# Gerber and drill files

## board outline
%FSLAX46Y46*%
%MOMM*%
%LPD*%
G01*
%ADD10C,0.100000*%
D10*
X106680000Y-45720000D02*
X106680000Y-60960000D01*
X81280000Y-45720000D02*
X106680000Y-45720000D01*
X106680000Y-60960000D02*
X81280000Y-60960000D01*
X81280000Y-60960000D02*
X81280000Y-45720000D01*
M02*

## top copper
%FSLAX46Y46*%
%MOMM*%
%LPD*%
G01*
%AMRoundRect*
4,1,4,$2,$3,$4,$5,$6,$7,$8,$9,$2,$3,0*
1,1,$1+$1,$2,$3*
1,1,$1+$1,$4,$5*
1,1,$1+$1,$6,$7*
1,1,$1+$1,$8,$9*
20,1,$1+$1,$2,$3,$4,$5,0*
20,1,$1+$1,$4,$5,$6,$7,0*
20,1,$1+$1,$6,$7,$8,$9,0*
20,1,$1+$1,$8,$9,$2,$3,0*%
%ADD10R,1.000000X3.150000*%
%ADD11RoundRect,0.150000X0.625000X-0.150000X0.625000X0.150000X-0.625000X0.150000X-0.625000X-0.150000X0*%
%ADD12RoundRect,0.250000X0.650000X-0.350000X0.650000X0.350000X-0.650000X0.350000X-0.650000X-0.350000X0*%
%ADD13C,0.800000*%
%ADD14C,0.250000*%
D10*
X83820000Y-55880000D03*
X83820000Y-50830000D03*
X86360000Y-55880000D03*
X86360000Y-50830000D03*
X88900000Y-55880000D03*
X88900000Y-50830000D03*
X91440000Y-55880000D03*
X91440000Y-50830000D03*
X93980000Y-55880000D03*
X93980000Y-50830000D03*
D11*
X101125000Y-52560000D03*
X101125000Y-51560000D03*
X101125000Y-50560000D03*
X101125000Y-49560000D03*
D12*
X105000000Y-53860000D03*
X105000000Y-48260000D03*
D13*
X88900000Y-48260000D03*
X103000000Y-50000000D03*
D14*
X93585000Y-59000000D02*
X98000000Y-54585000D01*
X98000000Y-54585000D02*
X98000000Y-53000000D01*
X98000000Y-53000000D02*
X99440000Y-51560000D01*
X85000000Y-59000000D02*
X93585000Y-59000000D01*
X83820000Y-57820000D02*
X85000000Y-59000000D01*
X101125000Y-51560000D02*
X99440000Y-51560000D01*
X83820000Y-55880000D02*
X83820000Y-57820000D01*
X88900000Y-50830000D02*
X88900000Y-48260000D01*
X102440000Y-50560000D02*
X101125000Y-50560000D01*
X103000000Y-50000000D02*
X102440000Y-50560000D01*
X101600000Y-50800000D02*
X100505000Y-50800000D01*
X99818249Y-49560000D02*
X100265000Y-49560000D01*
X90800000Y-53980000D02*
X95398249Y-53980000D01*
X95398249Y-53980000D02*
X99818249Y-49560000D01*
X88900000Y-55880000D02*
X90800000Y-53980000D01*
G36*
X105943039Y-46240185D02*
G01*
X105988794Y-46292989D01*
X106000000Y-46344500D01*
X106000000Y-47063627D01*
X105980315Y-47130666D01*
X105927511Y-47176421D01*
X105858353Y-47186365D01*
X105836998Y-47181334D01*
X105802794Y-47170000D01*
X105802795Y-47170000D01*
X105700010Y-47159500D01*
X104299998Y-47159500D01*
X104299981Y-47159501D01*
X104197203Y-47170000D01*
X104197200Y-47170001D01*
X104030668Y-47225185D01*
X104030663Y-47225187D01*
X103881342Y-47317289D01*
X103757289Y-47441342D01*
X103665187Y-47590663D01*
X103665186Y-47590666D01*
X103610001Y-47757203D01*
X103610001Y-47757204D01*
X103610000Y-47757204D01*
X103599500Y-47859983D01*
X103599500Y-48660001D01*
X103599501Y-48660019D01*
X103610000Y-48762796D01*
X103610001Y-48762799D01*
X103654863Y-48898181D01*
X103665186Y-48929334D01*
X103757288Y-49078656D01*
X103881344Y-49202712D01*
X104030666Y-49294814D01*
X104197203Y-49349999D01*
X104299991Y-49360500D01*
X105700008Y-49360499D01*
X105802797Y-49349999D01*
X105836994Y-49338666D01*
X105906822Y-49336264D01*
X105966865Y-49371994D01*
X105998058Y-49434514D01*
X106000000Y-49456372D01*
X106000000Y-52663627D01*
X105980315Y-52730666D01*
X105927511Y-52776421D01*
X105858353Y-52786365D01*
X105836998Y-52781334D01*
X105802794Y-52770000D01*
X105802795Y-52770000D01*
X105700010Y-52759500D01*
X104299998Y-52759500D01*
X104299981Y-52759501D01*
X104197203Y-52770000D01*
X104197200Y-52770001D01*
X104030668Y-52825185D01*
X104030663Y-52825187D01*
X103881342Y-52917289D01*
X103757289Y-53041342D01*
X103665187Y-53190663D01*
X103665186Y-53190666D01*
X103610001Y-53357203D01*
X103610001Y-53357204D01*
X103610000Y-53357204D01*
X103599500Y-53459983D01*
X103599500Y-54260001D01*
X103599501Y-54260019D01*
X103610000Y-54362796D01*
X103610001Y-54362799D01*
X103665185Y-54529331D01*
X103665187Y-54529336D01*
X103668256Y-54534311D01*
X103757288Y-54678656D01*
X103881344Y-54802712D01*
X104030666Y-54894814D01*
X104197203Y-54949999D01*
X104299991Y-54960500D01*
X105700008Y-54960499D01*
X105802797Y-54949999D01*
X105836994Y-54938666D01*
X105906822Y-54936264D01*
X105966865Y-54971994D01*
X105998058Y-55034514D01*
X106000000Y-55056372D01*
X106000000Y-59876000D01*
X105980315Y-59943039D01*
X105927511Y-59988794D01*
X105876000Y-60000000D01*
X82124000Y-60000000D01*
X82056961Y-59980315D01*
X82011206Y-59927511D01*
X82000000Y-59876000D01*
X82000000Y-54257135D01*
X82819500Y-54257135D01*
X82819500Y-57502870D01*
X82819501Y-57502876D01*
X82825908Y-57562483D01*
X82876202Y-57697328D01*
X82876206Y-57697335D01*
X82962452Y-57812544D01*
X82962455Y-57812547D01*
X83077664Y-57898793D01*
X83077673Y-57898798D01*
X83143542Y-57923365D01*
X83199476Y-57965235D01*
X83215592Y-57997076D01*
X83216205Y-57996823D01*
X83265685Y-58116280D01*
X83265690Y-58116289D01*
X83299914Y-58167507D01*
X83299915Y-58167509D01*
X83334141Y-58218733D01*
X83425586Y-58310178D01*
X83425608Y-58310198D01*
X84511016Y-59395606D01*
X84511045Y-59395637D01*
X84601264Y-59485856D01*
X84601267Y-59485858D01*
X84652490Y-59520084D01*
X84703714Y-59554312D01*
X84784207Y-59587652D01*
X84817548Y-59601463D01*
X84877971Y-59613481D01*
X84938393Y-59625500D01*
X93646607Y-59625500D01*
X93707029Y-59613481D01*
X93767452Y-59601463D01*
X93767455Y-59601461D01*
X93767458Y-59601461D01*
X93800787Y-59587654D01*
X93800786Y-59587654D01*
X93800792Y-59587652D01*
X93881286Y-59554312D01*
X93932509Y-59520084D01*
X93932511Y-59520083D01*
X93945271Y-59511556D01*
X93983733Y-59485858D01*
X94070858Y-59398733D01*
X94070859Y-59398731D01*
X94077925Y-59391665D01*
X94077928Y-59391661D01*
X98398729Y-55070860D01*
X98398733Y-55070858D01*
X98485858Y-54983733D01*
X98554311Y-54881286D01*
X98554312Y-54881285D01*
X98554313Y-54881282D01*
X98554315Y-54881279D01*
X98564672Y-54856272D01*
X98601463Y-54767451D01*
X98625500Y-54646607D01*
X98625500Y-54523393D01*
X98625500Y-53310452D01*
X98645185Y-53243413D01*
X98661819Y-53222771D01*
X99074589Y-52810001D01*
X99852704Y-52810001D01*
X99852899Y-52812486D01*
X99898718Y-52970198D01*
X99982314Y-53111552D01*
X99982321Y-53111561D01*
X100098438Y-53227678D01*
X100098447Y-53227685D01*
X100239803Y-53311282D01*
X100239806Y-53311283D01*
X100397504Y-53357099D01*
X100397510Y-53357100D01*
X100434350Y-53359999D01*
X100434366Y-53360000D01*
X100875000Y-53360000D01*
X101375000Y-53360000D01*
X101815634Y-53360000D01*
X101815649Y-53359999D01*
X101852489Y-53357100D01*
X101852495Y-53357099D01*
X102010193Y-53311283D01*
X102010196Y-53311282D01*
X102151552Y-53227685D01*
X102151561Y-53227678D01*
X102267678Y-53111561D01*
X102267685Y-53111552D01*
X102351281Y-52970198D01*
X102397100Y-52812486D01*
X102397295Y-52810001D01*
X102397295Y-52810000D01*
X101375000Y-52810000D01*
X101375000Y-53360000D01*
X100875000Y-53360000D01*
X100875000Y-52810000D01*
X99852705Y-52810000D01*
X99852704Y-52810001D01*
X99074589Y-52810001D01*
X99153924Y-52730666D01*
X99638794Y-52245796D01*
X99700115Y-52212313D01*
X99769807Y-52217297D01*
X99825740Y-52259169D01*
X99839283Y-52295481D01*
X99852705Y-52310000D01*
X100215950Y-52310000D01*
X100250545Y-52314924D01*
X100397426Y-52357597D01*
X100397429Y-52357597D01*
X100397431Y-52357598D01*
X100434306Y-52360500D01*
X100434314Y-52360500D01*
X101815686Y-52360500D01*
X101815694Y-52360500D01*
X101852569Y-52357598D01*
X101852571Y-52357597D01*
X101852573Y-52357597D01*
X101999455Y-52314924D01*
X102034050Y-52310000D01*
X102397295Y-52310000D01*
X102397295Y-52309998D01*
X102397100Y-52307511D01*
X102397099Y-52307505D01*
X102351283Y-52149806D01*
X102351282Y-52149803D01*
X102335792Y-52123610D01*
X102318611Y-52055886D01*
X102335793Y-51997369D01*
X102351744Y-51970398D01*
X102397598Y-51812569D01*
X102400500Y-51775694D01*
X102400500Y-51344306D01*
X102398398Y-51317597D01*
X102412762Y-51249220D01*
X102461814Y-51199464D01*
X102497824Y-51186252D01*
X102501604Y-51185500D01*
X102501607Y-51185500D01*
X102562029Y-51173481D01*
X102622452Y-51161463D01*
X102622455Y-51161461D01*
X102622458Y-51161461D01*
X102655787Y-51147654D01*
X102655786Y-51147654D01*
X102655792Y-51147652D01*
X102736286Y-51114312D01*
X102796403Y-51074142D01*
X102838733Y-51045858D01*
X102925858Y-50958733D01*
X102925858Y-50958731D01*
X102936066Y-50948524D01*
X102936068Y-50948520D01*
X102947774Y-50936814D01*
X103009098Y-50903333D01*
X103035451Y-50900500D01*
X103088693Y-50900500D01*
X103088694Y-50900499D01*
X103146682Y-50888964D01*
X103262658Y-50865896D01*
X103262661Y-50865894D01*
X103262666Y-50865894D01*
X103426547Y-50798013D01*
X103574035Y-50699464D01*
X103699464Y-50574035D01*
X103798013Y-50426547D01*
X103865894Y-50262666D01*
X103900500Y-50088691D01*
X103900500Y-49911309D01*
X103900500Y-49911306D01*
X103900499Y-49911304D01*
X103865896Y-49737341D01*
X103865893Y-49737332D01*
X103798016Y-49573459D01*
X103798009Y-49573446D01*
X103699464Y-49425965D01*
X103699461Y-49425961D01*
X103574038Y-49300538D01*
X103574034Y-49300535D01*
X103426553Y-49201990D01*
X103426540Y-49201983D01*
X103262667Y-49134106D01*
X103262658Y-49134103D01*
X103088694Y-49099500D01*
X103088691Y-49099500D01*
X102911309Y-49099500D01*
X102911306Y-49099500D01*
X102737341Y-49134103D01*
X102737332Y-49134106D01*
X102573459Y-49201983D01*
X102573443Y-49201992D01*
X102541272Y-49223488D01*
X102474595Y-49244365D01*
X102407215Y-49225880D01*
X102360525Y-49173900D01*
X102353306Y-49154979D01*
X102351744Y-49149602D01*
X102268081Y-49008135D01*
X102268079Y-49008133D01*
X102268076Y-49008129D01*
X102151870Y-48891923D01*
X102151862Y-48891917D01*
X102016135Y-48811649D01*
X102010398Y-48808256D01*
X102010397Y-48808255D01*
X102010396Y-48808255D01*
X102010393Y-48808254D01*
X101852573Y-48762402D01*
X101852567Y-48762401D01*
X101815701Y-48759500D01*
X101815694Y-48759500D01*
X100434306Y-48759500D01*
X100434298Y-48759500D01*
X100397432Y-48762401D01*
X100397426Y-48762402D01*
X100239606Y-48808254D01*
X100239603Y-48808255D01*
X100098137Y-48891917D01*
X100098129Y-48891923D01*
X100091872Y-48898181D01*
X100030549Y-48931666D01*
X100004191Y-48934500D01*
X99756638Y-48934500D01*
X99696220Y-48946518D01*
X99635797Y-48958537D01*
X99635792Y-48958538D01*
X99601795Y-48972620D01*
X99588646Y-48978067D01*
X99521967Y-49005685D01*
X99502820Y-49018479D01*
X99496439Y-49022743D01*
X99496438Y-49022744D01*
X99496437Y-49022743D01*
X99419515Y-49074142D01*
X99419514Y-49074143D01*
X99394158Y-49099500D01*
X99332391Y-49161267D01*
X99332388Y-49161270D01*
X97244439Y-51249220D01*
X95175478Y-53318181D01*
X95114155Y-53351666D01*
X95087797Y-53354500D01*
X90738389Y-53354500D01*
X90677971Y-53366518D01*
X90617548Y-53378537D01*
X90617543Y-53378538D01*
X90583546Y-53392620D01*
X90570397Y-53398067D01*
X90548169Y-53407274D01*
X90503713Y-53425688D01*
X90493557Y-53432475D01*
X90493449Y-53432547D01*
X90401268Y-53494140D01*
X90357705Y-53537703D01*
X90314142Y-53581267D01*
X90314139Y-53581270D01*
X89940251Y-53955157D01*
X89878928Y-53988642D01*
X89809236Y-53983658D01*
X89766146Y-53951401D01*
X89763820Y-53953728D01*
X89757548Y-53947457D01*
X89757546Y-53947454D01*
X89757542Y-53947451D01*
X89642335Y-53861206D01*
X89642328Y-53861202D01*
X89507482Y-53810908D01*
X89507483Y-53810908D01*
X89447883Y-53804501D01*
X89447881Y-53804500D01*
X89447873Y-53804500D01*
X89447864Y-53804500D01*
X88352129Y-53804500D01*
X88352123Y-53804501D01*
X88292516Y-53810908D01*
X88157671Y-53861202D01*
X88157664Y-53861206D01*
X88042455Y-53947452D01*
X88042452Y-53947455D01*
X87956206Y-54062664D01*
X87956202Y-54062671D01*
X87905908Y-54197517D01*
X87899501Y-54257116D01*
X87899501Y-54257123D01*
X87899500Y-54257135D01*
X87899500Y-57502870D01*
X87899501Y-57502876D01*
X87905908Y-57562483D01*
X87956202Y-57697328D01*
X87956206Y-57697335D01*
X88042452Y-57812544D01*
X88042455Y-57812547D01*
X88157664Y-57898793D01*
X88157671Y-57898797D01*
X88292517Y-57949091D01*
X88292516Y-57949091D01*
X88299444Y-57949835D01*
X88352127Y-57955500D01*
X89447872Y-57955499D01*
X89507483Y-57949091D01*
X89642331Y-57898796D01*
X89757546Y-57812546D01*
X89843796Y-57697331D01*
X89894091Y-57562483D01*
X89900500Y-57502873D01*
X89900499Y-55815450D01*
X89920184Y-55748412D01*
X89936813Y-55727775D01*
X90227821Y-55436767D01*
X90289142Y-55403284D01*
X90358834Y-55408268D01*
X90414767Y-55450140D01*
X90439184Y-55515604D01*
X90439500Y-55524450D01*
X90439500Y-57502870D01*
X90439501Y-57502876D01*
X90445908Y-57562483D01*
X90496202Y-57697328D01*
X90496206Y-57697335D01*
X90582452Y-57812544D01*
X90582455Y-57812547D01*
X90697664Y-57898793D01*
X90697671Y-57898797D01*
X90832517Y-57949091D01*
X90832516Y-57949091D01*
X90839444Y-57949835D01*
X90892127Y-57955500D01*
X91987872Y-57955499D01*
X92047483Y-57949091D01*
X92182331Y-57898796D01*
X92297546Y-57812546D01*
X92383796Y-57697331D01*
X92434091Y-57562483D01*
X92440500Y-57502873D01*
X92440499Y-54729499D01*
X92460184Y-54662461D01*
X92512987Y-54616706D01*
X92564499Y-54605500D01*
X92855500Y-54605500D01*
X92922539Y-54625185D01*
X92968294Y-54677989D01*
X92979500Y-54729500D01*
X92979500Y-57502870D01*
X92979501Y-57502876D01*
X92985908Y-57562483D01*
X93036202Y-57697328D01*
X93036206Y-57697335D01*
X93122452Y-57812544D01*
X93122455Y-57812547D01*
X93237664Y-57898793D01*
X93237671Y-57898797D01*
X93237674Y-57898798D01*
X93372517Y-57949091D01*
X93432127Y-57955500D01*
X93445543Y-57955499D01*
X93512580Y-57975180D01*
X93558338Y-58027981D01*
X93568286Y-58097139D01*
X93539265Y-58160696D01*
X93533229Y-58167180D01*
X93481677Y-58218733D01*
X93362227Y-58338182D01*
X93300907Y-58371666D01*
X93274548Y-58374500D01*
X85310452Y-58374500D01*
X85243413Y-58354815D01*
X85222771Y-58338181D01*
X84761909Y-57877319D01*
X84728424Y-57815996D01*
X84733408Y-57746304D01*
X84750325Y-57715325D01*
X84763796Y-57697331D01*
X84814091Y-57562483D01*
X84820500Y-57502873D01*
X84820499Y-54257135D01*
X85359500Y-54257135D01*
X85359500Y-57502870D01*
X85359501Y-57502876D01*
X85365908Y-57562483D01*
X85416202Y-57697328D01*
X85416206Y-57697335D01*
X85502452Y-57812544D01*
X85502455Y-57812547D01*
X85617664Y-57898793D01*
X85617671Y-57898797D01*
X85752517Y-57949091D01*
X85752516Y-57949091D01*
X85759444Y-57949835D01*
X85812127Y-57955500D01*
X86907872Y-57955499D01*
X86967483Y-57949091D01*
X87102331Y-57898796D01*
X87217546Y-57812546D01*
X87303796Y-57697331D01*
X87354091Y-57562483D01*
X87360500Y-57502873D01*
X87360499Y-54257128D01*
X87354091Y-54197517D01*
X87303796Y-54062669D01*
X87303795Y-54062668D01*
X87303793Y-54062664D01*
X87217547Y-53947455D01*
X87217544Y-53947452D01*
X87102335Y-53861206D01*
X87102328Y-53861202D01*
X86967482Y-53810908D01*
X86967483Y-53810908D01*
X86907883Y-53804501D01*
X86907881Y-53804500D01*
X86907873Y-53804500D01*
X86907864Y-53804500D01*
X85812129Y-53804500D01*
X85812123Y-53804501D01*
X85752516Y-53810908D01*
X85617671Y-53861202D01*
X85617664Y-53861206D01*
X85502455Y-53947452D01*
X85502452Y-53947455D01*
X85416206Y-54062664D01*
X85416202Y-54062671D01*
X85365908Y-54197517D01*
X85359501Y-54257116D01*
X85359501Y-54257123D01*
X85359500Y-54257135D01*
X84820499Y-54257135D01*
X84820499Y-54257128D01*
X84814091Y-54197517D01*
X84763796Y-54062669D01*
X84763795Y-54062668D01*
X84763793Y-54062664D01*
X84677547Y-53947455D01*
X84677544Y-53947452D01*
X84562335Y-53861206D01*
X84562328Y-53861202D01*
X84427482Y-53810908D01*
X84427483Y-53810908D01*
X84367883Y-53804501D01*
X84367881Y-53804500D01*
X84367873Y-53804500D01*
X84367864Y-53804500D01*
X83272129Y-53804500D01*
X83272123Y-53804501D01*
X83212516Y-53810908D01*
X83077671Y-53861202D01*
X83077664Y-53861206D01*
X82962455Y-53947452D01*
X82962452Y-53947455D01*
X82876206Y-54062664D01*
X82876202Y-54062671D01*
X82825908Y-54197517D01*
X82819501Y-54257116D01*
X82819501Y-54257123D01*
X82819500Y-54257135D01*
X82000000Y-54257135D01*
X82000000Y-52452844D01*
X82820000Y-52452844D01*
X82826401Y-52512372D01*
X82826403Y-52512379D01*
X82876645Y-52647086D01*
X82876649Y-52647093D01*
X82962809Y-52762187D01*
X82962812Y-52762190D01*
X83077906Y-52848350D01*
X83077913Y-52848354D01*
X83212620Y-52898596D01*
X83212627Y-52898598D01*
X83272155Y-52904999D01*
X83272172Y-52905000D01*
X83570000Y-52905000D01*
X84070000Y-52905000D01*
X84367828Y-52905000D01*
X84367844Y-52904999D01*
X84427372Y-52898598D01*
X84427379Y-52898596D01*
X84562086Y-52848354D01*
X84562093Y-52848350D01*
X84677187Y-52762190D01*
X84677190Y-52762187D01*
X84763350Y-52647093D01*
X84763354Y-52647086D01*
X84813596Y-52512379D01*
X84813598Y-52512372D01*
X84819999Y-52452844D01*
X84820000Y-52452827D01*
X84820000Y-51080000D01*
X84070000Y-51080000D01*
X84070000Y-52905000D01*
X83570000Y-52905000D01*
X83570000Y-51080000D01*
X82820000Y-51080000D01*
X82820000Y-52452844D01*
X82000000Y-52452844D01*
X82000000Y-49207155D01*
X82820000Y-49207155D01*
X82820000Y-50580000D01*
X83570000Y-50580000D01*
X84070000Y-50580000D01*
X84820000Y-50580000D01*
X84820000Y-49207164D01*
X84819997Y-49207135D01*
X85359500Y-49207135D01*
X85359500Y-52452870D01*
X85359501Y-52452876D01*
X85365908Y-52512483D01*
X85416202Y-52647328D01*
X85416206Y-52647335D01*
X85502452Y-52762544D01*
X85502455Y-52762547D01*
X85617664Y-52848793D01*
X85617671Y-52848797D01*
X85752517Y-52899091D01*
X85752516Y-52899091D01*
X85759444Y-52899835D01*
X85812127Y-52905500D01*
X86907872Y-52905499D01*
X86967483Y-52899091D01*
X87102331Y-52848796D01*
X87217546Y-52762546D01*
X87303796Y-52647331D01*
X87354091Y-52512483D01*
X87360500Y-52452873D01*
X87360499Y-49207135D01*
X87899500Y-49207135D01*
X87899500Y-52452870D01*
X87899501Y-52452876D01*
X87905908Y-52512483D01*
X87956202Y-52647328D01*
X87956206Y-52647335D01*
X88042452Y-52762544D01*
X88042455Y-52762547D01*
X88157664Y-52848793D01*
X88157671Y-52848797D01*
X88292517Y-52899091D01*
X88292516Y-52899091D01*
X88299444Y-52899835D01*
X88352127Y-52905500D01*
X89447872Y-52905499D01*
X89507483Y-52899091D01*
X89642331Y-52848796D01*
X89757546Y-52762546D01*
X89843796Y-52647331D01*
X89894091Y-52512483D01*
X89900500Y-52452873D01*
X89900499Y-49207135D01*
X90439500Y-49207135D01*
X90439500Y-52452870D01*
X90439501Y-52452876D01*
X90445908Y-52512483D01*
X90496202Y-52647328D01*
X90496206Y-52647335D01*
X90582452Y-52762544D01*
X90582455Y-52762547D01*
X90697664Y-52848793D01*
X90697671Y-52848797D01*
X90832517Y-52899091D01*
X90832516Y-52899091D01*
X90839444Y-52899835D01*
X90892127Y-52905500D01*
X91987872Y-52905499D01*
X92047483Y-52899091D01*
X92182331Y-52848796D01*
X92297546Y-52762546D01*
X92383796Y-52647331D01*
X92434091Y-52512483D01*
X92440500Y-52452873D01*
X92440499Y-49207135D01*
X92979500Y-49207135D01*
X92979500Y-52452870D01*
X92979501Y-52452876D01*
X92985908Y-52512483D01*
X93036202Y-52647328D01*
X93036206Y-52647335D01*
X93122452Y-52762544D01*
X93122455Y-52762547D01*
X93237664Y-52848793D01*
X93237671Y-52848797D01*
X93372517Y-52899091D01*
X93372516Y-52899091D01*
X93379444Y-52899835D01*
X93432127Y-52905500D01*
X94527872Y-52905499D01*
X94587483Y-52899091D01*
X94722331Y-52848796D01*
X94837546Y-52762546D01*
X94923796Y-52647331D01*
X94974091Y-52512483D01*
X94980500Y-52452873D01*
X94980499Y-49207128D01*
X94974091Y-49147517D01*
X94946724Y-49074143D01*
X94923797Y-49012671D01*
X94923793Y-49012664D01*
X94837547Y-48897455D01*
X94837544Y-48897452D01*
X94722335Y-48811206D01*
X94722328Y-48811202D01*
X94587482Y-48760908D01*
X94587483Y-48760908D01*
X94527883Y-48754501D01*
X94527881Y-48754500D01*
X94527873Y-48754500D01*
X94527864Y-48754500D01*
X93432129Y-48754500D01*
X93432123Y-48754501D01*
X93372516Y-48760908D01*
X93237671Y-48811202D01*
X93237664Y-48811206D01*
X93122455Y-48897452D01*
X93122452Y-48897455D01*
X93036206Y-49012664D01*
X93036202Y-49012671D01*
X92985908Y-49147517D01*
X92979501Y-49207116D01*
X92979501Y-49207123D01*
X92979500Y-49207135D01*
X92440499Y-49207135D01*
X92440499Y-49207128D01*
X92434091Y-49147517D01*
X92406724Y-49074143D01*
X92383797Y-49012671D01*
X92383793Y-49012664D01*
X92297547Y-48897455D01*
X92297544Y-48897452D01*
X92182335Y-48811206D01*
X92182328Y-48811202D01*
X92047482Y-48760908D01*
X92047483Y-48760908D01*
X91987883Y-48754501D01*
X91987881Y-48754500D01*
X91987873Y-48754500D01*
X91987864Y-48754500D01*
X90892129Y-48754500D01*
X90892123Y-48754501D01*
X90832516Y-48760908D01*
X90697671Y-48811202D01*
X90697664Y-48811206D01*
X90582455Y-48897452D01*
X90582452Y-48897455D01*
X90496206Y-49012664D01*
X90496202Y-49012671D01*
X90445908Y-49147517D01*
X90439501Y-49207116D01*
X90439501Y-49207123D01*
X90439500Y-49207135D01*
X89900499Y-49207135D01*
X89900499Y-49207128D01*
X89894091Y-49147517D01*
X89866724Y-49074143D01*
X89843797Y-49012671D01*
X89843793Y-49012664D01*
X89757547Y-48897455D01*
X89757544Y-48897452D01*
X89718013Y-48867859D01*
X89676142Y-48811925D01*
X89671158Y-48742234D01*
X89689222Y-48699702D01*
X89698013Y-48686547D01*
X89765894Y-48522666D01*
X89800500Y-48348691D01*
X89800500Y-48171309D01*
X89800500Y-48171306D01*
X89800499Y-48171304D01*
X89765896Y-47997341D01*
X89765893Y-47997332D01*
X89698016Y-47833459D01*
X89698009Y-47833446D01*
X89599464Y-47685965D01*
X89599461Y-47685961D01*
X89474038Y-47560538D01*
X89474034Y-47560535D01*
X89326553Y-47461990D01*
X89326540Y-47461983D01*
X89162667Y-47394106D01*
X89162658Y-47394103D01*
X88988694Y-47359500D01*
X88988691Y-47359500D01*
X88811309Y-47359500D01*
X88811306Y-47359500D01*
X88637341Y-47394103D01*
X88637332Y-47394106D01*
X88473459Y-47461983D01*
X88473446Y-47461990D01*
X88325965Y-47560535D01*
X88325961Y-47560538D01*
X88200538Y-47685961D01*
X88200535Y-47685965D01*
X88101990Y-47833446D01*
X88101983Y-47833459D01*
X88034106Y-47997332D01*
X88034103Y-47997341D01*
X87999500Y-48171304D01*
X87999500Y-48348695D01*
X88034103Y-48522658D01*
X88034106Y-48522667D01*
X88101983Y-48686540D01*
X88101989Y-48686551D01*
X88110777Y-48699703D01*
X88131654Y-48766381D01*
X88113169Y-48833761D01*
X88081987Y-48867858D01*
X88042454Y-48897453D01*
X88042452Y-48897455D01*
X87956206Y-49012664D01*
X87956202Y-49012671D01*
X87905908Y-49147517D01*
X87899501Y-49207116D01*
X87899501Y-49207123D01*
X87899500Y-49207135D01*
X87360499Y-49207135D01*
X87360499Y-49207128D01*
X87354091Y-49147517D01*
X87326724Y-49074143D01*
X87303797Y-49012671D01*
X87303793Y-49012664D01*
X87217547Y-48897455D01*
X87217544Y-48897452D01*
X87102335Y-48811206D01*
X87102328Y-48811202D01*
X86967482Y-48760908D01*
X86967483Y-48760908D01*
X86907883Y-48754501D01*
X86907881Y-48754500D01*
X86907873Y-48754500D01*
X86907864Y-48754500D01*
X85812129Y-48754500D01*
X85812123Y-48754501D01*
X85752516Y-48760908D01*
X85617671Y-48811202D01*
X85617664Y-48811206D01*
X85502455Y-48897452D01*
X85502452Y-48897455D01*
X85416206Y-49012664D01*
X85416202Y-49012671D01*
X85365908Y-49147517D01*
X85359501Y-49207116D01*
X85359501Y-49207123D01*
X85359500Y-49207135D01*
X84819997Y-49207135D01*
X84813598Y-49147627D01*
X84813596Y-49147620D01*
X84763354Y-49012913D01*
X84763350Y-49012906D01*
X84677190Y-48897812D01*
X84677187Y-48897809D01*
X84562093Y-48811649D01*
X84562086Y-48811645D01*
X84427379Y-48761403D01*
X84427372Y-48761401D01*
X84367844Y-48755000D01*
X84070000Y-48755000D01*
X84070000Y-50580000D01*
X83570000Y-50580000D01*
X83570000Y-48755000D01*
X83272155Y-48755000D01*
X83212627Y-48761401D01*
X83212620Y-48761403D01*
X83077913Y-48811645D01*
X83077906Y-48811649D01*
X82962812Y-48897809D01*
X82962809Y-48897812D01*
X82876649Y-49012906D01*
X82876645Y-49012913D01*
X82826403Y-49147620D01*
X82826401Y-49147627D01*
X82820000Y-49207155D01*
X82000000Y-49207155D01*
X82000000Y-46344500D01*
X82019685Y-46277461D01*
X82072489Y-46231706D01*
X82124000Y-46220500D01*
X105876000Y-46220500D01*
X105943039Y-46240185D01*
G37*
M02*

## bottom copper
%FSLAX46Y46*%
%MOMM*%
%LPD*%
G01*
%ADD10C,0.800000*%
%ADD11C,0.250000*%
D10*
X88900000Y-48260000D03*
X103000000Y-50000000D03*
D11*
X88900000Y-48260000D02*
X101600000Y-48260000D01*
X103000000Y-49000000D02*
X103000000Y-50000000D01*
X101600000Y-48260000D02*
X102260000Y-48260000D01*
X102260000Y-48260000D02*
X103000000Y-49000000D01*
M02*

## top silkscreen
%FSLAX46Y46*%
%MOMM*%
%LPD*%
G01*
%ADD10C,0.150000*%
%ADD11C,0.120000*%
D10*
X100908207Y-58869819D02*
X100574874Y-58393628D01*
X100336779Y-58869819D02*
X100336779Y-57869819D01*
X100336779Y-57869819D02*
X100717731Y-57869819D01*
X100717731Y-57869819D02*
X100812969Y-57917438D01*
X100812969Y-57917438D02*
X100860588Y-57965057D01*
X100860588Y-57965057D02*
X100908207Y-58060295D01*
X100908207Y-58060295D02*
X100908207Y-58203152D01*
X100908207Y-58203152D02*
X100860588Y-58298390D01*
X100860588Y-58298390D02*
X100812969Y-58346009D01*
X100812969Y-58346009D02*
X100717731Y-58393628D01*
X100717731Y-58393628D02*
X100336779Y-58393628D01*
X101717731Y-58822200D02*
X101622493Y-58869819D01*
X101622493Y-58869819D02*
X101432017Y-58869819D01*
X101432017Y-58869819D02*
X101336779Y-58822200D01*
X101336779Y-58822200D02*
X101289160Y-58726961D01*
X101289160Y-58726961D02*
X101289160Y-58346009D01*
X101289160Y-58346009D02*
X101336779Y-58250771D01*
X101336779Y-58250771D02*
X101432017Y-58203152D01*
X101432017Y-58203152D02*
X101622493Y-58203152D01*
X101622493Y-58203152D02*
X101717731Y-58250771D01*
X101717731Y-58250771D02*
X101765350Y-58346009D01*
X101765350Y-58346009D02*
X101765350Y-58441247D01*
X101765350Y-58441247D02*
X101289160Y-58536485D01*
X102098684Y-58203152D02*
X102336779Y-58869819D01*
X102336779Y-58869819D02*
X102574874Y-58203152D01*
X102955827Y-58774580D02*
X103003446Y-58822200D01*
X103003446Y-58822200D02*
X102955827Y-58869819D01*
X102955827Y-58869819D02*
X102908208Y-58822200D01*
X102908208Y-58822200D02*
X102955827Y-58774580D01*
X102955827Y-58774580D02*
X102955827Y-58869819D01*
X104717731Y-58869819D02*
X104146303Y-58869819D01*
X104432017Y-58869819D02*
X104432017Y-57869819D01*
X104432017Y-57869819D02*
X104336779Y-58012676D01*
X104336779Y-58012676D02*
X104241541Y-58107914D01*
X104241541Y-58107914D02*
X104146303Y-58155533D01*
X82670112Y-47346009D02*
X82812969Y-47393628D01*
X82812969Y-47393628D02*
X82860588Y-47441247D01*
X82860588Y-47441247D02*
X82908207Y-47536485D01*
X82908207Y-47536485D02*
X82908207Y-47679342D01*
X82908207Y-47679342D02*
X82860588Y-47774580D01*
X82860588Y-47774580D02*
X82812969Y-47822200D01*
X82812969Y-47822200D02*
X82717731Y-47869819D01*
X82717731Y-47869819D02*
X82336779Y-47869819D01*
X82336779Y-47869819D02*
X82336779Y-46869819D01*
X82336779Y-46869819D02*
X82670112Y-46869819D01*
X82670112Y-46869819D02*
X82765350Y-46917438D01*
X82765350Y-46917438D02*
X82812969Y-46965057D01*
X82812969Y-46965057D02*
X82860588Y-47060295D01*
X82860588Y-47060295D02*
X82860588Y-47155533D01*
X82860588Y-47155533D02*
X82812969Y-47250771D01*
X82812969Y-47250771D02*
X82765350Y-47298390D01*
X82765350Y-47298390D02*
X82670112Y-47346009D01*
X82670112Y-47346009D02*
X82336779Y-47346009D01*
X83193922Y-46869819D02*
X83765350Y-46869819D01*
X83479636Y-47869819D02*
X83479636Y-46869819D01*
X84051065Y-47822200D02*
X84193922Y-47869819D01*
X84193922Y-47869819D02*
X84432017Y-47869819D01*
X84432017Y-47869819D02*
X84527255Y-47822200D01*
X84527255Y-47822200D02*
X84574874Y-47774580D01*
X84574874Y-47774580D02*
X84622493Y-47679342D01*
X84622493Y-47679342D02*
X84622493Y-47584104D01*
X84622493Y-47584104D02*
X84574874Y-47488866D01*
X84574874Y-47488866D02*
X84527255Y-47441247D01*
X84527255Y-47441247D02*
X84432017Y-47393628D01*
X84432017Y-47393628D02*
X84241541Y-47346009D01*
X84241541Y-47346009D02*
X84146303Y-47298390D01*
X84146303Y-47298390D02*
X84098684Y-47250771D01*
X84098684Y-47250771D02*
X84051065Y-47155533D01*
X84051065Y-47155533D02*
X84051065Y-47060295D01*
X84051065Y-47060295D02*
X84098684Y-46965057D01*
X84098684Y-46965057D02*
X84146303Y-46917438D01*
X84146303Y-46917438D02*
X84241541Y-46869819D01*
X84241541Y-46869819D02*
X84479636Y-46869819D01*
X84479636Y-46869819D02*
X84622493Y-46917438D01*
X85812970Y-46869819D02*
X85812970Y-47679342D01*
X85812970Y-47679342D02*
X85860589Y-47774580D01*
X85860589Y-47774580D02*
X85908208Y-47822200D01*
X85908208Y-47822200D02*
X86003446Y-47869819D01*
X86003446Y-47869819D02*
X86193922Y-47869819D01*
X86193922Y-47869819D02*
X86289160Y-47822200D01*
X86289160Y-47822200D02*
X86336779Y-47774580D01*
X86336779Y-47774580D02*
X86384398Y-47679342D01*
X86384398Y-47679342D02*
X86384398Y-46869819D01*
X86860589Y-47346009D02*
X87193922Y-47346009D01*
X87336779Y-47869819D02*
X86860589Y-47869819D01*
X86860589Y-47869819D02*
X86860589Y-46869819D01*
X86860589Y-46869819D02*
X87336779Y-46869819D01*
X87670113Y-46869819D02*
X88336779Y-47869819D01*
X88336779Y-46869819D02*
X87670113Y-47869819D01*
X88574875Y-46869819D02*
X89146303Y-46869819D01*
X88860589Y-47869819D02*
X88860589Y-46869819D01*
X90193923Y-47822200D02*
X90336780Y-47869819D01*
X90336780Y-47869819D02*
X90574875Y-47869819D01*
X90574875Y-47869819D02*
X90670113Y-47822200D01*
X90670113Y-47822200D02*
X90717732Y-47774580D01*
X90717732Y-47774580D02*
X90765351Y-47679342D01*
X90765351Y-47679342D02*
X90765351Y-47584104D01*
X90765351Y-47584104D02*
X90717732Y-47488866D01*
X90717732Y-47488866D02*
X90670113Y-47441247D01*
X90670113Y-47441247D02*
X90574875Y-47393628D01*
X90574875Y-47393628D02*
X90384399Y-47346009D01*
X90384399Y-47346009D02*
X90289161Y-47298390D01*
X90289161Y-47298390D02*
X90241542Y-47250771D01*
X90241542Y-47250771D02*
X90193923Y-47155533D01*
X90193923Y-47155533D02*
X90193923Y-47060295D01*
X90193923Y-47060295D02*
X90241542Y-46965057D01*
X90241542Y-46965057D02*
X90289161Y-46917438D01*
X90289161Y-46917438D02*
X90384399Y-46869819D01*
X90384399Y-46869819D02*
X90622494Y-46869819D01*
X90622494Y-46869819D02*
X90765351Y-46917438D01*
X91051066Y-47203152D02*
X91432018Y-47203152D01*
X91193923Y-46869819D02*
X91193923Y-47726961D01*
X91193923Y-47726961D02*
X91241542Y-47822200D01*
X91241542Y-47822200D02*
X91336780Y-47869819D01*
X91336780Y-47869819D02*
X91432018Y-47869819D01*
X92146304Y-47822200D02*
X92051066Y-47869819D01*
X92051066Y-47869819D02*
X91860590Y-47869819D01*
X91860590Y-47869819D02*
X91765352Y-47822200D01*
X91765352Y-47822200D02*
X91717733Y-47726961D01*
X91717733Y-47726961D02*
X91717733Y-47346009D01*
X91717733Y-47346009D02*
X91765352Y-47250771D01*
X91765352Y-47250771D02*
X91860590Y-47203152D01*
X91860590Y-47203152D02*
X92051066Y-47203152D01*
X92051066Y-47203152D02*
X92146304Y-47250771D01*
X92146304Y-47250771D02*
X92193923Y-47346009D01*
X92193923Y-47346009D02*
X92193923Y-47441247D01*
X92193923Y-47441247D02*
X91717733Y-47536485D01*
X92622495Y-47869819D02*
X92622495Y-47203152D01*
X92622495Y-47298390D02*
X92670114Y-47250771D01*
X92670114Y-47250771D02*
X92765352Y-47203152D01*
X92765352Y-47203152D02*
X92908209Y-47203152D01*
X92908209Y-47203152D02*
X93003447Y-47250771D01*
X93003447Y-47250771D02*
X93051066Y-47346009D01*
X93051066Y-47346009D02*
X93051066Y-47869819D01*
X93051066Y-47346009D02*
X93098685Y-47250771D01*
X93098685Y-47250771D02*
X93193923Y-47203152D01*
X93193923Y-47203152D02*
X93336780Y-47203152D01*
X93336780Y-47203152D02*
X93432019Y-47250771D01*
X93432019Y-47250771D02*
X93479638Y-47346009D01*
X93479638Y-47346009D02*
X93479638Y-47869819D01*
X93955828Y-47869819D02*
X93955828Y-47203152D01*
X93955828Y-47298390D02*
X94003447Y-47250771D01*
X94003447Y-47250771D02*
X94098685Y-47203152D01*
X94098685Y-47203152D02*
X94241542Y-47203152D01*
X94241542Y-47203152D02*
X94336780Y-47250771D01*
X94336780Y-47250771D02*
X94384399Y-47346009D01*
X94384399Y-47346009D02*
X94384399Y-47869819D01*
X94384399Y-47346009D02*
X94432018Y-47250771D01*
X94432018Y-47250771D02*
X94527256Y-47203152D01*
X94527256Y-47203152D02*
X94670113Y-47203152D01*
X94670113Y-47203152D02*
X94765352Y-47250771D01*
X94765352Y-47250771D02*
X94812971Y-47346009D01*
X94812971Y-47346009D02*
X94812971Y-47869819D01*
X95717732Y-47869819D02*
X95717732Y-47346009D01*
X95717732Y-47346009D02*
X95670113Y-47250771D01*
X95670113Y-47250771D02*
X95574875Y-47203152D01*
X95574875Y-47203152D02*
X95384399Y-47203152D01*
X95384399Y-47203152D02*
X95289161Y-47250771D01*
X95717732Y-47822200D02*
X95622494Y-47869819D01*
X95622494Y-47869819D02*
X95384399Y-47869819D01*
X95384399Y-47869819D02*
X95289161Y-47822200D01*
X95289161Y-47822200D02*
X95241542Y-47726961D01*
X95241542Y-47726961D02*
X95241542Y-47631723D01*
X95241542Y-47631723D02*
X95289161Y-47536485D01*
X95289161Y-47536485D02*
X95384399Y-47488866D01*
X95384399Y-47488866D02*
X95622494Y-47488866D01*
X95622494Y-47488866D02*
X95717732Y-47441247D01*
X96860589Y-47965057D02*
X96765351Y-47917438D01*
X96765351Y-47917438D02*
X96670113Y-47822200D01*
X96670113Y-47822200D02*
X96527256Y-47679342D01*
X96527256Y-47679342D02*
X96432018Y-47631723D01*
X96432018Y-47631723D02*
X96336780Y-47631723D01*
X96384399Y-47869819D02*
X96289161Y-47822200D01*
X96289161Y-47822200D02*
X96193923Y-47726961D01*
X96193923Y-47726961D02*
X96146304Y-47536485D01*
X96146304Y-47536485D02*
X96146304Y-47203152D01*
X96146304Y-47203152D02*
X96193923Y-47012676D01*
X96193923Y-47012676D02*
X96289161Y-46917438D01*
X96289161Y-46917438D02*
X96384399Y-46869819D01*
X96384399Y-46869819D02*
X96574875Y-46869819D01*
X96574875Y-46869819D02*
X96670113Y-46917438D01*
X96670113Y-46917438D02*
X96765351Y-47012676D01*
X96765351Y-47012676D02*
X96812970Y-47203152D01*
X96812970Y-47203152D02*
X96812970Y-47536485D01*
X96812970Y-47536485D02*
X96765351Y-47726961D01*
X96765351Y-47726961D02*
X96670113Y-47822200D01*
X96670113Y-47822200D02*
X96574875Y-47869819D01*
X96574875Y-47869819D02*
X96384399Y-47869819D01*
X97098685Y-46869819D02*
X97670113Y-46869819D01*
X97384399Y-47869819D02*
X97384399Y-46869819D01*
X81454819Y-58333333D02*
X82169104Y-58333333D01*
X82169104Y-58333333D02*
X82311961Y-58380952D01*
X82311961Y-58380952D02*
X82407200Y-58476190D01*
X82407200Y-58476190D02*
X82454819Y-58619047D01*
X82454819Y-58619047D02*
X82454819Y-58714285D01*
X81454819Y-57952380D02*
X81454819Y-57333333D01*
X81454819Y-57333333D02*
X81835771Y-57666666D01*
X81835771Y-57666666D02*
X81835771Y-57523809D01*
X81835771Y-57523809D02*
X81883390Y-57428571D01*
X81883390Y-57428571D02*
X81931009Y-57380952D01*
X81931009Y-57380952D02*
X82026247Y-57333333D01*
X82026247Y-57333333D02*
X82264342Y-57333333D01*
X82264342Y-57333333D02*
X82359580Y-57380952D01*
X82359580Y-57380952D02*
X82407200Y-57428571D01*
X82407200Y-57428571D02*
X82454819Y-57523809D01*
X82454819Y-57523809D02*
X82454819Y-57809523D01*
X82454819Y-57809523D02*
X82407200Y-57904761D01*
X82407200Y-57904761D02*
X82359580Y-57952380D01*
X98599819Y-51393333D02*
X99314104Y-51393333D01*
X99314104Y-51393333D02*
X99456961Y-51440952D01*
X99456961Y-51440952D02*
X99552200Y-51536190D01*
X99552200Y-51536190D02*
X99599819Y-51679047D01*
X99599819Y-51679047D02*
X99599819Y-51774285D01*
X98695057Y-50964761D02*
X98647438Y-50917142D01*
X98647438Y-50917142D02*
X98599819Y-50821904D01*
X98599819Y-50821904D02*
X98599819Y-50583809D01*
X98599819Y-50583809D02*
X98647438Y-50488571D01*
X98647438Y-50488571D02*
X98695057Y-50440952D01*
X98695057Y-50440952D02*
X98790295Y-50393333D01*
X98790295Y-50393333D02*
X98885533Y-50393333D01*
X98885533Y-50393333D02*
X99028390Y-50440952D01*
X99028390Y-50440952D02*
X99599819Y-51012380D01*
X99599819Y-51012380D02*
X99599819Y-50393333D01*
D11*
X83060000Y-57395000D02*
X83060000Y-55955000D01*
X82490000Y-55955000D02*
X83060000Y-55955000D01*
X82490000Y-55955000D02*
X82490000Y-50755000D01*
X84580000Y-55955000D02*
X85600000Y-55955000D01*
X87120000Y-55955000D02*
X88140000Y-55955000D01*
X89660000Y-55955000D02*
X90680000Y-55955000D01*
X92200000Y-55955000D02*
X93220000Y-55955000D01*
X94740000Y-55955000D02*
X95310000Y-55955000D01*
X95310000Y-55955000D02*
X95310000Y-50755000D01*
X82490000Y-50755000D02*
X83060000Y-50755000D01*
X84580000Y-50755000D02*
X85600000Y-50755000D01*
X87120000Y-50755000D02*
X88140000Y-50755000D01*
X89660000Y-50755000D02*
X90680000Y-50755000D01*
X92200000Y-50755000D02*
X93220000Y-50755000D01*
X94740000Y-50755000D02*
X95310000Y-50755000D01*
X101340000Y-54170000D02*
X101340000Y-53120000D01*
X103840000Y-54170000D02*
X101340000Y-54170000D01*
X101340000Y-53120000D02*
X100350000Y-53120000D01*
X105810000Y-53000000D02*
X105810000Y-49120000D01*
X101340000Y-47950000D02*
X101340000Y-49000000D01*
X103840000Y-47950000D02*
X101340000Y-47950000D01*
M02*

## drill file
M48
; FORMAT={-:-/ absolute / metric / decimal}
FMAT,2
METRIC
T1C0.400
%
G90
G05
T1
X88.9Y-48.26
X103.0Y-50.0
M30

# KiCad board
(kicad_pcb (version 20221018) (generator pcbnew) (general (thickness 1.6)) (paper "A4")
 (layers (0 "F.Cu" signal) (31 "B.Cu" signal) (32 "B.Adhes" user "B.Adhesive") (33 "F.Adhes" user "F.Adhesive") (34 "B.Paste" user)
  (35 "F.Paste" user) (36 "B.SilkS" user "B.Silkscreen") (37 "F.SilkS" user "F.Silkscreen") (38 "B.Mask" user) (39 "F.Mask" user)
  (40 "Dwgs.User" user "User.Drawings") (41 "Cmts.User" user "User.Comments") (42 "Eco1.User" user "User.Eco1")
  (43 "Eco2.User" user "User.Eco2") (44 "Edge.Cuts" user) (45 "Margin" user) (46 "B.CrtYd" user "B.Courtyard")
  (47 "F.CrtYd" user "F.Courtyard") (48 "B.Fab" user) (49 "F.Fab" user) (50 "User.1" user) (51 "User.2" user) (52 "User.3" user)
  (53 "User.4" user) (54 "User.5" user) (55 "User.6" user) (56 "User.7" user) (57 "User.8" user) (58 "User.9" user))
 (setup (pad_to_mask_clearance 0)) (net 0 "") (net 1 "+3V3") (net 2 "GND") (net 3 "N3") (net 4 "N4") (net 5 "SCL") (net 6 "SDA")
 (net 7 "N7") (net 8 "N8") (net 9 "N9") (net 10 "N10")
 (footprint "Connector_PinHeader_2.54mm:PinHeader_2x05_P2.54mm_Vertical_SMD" (layer "F.Cu") (at 88.9 53.355 90)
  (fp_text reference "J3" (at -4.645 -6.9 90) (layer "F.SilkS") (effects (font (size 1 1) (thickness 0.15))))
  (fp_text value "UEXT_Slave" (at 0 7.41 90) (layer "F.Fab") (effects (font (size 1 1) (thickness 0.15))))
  (fp_line (start -4.04 -5.84) (end -2.6 -5.84) (stroke (width 0.12) (type solid)) (layer "F.SilkS"))
  (fp_line (start -2.6 -6.41) (end -2.6 -5.84) (stroke (width 0.12) (type solid)) (layer "F.SilkS"))
  (fp_line (start -2.6 -6.41) (end 2.6 -6.41) (stroke (width 0.12) (type solid)) (layer "F.SilkS"))
  (fp_line (start -2.6 -4.32) (end -2.6 -3.3) (stroke (width 0.12) (type solid)) (layer "F.SilkS"))
  (fp_line (start -2.6 -1.78) (end -2.6 -0.76) (stroke (width 0.12) (type solid)) (layer "F.SilkS"))
  (fp_line (start -2.6 0.76) (end -2.6 1.78) (stroke (width 0.12) (type solid)) (layer "F.SilkS"))
  (fp_line (start -2.6 3.3) (end -2.6 4.32) (stroke (width 0.12) (type solid)) (layer "F.SilkS"))
  (fp_line (start -2.6 5.84) (end -2.6 6.41) (stroke (width 0.12) (type solid)) (layer "F.SilkS"))
  (fp_line (start -2.6 6.41) (end 2.6 6.41) (stroke (width 0.12) (type solid)) (layer "F.SilkS"))
  (fp_line (start 2.6 -6.41) (end 2.6 -5.84) (stroke (width 0.12) (type solid)) (layer "F.SilkS"))
  (fp_line (start 2.6 -4.32) (end 2.6 -3.3) (stroke (width 0.12) (type solid)) (layer "F.SilkS"))
  (fp_line (start 2.6 -1.78) (end 2.6 -0.76) (stroke (width 0.12) (type solid)) (layer "F.SilkS"))
  (fp_line (start 2.6 0.76) (end 2.6 1.78) (stroke (width 0.12) (type solid)) (layer "F.SilkS"))
  (fp_line (start 2.6 3.3) (end 2.6 4.32) (stroke (width 0.12) (type solid)) (layer "F.SilkS"))
  (fp_line (start 2.6 5.84) (end 2.6 6.41) (stroke (width 0.12) (type solid)) (layer "F.SilkS"))
  (pad "1" smd rect (at -2.525 -5.08 90) (size 3.15 1) (layers "F.Cu" "F.Paste" "F.Mask") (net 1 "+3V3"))
  (pad "2" smd rect (at 2.525 -5.08 90) (size 3.15 1) (layers "F.Cu" "F.Paste" "F.Mask") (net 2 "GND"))
  (pad "3" smd rect (at -2.525 -2.54 90) (size 3.15 1) (layers "F.Cu" "F.Paste" "F.Mask") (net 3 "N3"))
  (pad "4" smd rect (at 2.525 -2.54 90) (size 3.15 1) (layers "F.Cu" "F.Paste" "F.Mask") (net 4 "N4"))
  (pad "5" smd rect (at -2.525 0 90) (size 3.15 1) (layers "F.Cu" "F.Paste" "F.Mask") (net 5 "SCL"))
  (pad "6" smd rect (at 2.525 0 90) (size 3.15 1) (layers "F.Cu" "F.Paste" "F.Mask") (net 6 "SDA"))
  (pad "7" smd rect (at -2.525 2.54 90) (size 3.15 1) (layers "F.Cu" "F.Paste" "F.Mask") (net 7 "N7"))
  (pad "8" smd rect (at 2.525 2.54 90) (size 3.15 1) (layers "F.Cu" "F.Paste" "F.Mask") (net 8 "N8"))
  (pad "9" smd rect (at -2.525 5.08 90) (size 3.15 1) (layers "F.Cu" "F.Paste" "F.Mask") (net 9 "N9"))
  (pad "10" smd rect (at 2.525 5.08 90) (size 3.15 1) (layers "F.Cu" "F.Paste" "F.Mask") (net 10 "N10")))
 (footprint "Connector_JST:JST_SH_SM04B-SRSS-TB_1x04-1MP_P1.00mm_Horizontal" (layer "F.Cu") (at 103.125 51.06 90)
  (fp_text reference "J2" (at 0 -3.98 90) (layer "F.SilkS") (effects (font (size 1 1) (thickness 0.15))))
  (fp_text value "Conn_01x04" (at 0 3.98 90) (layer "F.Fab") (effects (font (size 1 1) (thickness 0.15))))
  (fp_line (start -3.11 -1.785) (end -2.06 -1.785) (stroke (width 0.12) (type solid)) (layer "F.SilkS"))
  (fp_line (start -3.11 0.715) (end -3.11 -1.785) (stroke (width 0.12) (type solid)) (layer "F.SilkS"))
  (fp_line (start -2.06 -1.785) (end -2.06 -2.775) (stroke (width 0.12) (type solid)) (layer "F.SilkS"))
  (fp_line (start -1.94 2.685) (end 1.94 2.685) (stroke (width 0.12) (type solid)) (layer "F.SilkS"))
  (fp_line (start 3.11 -1.785) (end 2.06 -1.785) (stroke (width 0.12) (type solid)) (layer "F.SilkS"))
  (fp_line (start 3.11 0.715) (end 3.11 -1.785) (stroke (width 0.12) (type solid)) (layer "F.SilkS"))
  (pad "1" smd roundrect (at -1.5 -2 90) (size 0.6 1.55) (layers "F.Cu" "F.Paste" "F.Mask") (roundrect_rratio 0.25) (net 2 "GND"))
  (pad "2" smd roundrect (at -0.5 -2 90) (size 0.6 1.55) (layers "F.Cu" "F.Paste" "F.Mask") (roundrect_rratio 0.25) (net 1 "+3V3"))
  (pad "3" smd roundrect (at 0.5 -2 90) (size 0.6 1.55) (layers "F.Cu" "F.Paste" "F.Mask") (roundrect_rratio 0.25) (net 6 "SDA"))
  (pad "4" smd roundrect (at 1.5 -2 90) (size 0.6 1.55) (layers "F.Cu" "F.Paste" "F.Mask") (roundrect_rratio 0.25) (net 5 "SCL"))
  (pad "MP" smd roundrect (at -2.8 1.875 90) (size 1.2 1.8) (layers "F.Cu" "F.Paste" "F.Mask") (roundrect_rratio 0.2083333333))
  (pad "MP" smd roundrect (at 2.8 1.875 90) (size 1.2 1.8) (layers "F.Cu" "F.Paste" "F.Mask") (roundrect_rratio 0.2083333333)))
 (gr_line (start 106.68 45.72) (end 106.68 60.96) (stroke (width 0.1) (type default)) (layer "Edge.Cuts"))
 (gr_line (start 81.28 45.72) (end 106.68 45.72) (stroke (width 0.1) (type default)) (layer "Edge.Cuts"))
 (gr_line (start 106.68 60.96) (end 81.28 60.96) (stroke (width 0.1) (type default)) (layer "Edge.Cuts"))
 (gr_line (start 81.28 60.96) (end 81.28 45.72) (stroke (width 0.1) (type default)) (layer "Edge.Cuts"))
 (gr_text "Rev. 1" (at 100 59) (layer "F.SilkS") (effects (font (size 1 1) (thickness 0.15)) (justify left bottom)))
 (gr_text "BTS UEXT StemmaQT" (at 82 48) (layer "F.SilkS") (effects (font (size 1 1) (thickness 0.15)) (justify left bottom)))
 (segment (start 93.585 59) (end 98 54.585) (width 0.25) (layer "F.Cu") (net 1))
 (segment (start 98 54.585) (end 98 53) (width 0.25) (layer "F.Cu") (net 1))
 (segment (start 98 53) (end 99.44 51.56) (width 0.25) (layer "F.Cu") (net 1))
 (segment (start 85 59) (end 93.585 59) (width 0.25) (layer "F.Cu") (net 1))
 (segment (start 83.82 57.82) (end 85 59) (width 0.25) (layer "F.Cu") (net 1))
 (segment (start 101.125 51.56) (end 99.44 51.56) (width 0.25) (layer "F.Cu") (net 1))
 (segment (start 83.82 55.88) (end 83.82 57.82) (width 0.25) (layer "F.Cu") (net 1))
 (segment (start 88.9 50.83) (end 88.9 48.26) (width 0.25) (layer "F.Cu") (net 6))
 (segment (start 102.44 50.56) (end 101.125 50.56) (width 0.25) (layer "F.Cu") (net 6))
 (segment (start 103 50) (end 102.44 50.56) (width 0.25) (layer "F.Cu") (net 6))
 (segment (start 101.6 50.8) (end 100.505 50.8) (width 0.25) (layer "F.Cu") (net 6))
 (via (at 88.9 48.26) (size 0.8) (drill 0.4) (layers "F.Cu" "B.Cu") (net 6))
 (via (at 103 50) (size 0.8) (drill 0.4) (layers "F.Cu" "B.Cu") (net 6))
 (segment (start 88.9 48.26) (end 101.6 48.26) (width 0.25) (layer "B.Cu") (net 6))
 (segment (start 103 49) (end 103 50) (width 0.25) (layer "B.Cu") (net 6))
 (segment (start 101.6 48.26) (end 102.26 48.26) (width 0.25) (layer "B.Cu") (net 6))
 (segment (start 102.26 48.26) (end 103 49) (width 0.25) (layer "B.Cu") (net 6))
 (segment (start 99.818249 49.56) (end 100.265 49.56) (width 0.25) (layer "F.Cu") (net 5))
 (segment (start 90.8 53.98) (end 95.398249 53.98) (width 0.25) (layer "F.Cu") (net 5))
 (segment (start 95.398249 53.98) (end 99.818249 49.56) (width 0.25) (layer "F.Cu") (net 5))
 (segment (start 88.9 55.88) (end 90.8 53.98) (width 0.25) (layer "F.Cu") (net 5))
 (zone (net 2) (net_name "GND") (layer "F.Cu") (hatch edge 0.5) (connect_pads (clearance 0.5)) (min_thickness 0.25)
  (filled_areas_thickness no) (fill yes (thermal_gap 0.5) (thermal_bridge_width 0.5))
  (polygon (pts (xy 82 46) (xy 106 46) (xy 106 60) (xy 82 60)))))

